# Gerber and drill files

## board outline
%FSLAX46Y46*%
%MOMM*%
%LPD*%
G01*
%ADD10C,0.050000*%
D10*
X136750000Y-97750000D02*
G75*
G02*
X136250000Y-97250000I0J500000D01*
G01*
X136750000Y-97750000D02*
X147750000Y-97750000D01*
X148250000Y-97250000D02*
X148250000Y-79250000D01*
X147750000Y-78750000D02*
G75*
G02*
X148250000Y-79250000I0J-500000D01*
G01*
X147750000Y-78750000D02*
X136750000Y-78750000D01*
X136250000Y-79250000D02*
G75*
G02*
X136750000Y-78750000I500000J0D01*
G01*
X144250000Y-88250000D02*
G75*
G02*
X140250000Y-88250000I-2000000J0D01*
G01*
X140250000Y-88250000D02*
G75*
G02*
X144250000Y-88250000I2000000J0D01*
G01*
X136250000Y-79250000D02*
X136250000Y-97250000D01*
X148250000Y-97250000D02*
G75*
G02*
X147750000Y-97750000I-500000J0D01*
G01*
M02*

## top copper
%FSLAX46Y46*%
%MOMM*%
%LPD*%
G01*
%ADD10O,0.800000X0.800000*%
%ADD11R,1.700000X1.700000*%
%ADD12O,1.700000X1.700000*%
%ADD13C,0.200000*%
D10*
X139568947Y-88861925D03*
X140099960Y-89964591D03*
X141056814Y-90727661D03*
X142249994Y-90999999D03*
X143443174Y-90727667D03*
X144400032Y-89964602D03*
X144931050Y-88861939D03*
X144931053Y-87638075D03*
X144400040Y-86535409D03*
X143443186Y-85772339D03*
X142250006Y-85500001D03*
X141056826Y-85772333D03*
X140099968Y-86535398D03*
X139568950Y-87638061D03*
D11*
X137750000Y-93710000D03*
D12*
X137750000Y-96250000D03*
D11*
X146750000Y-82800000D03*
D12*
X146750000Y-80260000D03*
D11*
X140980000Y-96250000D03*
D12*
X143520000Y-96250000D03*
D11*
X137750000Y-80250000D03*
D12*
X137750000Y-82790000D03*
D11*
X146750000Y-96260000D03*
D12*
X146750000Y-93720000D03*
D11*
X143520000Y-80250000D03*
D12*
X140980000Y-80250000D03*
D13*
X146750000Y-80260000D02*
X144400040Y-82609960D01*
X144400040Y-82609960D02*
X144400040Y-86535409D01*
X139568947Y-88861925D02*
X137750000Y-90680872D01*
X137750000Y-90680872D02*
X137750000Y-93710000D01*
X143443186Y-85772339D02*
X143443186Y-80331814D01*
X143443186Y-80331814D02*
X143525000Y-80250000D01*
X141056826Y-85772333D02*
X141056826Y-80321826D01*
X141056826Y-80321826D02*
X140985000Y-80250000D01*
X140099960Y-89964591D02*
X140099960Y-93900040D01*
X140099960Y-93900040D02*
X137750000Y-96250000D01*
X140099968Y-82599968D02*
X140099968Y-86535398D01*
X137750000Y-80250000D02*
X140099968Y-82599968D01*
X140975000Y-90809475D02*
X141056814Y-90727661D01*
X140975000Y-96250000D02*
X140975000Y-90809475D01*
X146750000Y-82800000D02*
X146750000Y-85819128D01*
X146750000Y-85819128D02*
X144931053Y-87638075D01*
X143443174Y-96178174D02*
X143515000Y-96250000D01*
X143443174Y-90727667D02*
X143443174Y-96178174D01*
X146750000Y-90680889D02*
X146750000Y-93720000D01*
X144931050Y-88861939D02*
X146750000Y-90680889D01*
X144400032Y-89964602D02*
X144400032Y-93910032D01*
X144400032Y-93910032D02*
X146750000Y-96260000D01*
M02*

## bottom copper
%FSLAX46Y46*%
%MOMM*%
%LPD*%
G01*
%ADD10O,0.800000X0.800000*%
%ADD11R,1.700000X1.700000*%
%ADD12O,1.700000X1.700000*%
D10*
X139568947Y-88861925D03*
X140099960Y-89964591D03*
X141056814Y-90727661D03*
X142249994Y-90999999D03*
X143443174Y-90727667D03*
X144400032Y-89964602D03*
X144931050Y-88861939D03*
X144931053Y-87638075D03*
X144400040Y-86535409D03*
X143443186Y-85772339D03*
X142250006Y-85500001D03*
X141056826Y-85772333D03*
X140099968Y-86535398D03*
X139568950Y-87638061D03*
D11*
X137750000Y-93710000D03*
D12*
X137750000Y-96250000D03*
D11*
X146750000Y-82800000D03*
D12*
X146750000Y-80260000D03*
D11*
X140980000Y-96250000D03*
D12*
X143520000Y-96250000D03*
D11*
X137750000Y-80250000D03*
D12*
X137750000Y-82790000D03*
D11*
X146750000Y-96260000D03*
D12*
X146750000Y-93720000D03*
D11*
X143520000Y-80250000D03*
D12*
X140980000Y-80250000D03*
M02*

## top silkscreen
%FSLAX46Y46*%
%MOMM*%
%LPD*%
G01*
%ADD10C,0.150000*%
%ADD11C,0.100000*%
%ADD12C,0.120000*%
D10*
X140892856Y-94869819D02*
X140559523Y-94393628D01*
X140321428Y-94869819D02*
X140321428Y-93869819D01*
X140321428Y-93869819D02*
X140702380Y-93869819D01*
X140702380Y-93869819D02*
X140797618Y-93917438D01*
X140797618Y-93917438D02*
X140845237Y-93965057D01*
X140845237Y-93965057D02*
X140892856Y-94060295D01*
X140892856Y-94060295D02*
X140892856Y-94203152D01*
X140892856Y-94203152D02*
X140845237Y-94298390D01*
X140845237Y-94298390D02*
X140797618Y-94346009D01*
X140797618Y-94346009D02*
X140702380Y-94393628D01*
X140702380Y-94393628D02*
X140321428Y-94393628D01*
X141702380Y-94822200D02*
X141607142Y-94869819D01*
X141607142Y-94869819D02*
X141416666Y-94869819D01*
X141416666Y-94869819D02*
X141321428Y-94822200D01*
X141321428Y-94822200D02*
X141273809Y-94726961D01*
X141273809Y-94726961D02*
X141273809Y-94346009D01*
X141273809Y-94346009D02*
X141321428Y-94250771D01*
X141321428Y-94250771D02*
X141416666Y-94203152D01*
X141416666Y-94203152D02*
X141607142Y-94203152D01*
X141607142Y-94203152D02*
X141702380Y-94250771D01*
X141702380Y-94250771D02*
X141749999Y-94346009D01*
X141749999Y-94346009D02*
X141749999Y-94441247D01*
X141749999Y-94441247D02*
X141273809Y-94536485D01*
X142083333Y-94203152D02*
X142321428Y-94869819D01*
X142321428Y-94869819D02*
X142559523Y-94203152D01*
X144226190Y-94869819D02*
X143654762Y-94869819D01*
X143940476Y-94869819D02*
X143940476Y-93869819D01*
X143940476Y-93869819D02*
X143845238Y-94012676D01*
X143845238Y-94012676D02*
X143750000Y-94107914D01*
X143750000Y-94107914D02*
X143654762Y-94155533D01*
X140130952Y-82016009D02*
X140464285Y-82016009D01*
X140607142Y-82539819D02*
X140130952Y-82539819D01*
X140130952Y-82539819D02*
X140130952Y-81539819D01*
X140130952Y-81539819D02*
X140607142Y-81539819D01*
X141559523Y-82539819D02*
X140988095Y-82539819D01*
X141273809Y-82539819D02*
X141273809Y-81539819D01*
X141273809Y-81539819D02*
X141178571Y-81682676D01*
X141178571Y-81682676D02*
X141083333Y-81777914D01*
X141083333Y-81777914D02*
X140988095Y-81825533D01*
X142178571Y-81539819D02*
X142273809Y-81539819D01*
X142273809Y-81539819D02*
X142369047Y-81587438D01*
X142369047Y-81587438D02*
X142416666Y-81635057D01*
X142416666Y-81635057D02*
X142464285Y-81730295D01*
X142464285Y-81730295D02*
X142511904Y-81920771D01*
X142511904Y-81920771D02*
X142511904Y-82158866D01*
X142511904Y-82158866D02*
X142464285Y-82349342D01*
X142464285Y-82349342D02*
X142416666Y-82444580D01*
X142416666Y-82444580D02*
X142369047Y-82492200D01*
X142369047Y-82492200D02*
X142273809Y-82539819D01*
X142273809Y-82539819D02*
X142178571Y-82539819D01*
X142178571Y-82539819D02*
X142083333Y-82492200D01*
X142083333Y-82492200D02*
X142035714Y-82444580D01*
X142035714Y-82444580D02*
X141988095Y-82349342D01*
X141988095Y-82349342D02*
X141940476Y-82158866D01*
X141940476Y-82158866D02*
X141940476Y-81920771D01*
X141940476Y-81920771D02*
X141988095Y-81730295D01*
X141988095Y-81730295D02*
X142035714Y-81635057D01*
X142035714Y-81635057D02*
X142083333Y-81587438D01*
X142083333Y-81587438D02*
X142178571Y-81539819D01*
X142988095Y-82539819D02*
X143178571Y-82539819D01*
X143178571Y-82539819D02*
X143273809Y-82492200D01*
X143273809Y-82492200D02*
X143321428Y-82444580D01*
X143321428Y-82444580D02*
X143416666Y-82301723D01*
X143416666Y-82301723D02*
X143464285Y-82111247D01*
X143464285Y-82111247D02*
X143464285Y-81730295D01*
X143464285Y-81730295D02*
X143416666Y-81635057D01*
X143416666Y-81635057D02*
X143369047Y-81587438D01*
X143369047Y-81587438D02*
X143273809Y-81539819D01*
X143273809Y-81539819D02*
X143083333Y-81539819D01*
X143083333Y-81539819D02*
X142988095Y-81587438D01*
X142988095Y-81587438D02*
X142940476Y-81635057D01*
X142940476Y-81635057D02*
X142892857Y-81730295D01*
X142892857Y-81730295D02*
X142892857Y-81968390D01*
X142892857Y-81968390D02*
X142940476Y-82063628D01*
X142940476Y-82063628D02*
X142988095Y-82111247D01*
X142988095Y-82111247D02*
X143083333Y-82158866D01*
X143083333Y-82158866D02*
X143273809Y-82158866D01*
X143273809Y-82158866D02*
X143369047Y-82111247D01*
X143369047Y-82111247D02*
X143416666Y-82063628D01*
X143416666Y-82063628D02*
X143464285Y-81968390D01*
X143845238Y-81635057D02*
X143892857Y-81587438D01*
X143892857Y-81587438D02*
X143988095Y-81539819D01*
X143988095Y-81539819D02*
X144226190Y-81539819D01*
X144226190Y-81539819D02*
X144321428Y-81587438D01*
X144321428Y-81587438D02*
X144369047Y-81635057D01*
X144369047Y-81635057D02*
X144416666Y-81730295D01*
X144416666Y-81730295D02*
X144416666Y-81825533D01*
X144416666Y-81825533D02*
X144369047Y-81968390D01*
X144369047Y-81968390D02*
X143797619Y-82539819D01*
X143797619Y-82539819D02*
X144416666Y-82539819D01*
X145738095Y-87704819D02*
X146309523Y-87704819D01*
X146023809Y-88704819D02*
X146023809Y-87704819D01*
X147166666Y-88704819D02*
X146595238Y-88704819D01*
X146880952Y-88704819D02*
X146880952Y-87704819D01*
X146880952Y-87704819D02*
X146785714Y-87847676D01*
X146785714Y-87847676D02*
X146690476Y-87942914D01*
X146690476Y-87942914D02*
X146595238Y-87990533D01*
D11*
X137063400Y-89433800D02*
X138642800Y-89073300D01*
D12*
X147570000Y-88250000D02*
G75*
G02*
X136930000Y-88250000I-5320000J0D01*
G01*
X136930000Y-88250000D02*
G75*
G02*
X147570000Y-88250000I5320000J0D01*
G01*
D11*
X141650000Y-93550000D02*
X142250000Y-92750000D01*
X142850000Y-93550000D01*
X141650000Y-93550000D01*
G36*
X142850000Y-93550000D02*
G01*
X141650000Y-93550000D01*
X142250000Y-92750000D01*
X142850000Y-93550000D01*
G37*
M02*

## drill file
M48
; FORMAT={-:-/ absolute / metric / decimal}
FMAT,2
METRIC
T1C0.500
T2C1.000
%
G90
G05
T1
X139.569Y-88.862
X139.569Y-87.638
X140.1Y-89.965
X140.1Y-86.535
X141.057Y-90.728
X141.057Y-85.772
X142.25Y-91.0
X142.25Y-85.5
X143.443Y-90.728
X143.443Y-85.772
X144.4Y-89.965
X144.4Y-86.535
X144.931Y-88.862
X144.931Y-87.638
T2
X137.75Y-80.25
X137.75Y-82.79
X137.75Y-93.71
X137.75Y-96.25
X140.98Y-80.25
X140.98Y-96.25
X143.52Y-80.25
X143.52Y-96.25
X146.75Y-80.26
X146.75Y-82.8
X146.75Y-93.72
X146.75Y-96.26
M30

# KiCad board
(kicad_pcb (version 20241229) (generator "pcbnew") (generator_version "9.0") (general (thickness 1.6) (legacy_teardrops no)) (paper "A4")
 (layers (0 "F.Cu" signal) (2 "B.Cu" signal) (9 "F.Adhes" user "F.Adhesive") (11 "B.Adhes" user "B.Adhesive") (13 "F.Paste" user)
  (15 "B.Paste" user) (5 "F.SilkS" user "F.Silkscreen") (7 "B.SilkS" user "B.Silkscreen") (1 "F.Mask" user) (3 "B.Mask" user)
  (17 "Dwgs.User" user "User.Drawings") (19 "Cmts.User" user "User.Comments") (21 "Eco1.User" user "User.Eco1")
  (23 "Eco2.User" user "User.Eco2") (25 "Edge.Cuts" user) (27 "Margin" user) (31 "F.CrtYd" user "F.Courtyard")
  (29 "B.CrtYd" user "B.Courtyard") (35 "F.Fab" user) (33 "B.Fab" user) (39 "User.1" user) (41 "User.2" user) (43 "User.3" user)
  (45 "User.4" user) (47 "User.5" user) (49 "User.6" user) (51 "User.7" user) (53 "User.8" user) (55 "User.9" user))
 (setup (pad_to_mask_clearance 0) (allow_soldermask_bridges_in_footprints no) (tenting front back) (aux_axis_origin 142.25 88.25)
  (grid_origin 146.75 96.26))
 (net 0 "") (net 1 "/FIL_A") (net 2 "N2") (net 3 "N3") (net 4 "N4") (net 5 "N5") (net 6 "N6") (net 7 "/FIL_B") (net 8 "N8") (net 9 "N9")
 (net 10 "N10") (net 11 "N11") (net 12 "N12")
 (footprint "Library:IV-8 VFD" (layer "F.Cu") (at 142.25 88.25)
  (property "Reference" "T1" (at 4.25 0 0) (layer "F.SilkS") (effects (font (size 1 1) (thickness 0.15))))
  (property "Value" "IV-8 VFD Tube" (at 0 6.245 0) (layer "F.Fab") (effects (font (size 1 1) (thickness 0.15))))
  (fp_line (start -5.1866 1.1838) (end -3.6072 0.8233) (stroke (width 0.1) (type default)) (layer "F.SilkS"))
  (fp_circle (center 0 0) (end 0 5.32) (stroke (width 0.12) (type default)) (fill no) (layer "F.SilkS"))
  (fp_poly (pts (xy -0.6 5.3) (xy 0 4.5) (xy 0.6 5.3)) (stroke (width 0.1) (type solid)) (fill yes) (layer "F.SilkS"))
  (pad "1" thru_hole oval (at -2.681053 0.611925) (size 0.8 0.8) (drill 0.5) (layers "*.Cu" "*.Mask") (remove_unused_layers no)
   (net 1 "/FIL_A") (thermal_bridge_angle 45))
  (pad "2" thru_hole oval (at -2.15004 1.714591) (size 0.8 0.8) (drill 0.5) (layers "*.Cu" "*.Mask") (remove_unused_layers no) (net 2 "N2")
   (thermal_bridge_angle 45))
  (pad "3" thru_hole oval (at -1.193186 2.477661) (size 0.8 0.8) (drill 0.5) (layers "*.Cu" "*.Mask") (remove_unused_layers no) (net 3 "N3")
   (thermal_bridge_angle 45))
  (pad "4" thru_hole oval (at -0.000006 2.749999) (size 0.8 0.8) (drill 0.5) (layers "*.Cu" "*.Mask") (remove_unused_layers no)
   (thermal_bridge_angle 45))
  (pad "5" thru_hole oval (at 1.193174 2.477667) (size 0.8 0.8) (drill 0.5) (layers "*.Cu" "*.Mask") (remove_unused_layers no) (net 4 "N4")
   (thermal_bridge_angle 45))
  (pad "6" thru_hole oval (at 2.150032 1.714602) (size 0.8 0.8) (drill 0.5) (layers "*.Cu" "*.Mask") (remove_unused_layers no) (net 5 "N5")
   (thermal_bridge_angle 45))
  (pad "7" thru_hole oval (at 2.68105 0.611939) (size 0.8 0.8) (drill 0.5) (layers "*.Cu" "*.Mask") (remove_unused_layers no) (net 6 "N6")
   (thermal_bridge_angle 45))
  (pad "8" thru_hole oval (at 2.681053 -0.611925) (size 0.8 0.8) (drill 0.5) (layers "*.Cu" "*.Mask") (remove_unused_layers no)
   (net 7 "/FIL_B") (thermal_bridge_angle 45))
  (pad "9" thru_hole oval (at 2.15004 -1.714591) (size 0.8 0.8) (drill 0.5) (layers "*.Cu" "*.Mask") (remove_unused_layers no) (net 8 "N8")
   (thermal_bridge_angle 45))
  (pad "10" thru_hole oval (at 1.193186 -2.477661) (size 0.8 0.8) (drill 0.5) (layers "*.Cu" "*.Mask") (remove_unused_layers no)
   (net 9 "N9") (thermal_bridge_angle 45))
  (pad "11" thru_hole oval (at 0.000006 -2.749999) (size 0.8 0.8) (drill 0.5) (layers "*.Cu" "*.Mask") (remove_unused_layers no)
   (thermal_bridge_angle 45))
  (pad "12" thru_hole oval (at -1.193174 -2.477667) (size 0.8 0.8) (drill 0.5) (layers "*.Cu" "*.Mask") (remove_unused_layers no)
   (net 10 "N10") (thermal_bridge_angle 45))
  (pad "13" thru_hole oval (at -2.150032 -1.714602) (size 0.8 0.8) (drill 0.5) (layers "*.Cu" "*.Mask") (remove_unused_layers no)
   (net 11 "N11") (thermal_bridge_angle 45))
  (pad "14" thru_hole oval (at -2.68105 -0.611939) (size 0.8 0.8) (drill 0.5) (layers "*.Cu" "*.Mask") (remove_unused_layers no)
   (thermal_bridge_angle 45)))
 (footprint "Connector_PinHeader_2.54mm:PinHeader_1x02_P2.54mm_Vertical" (layer "B.Cu") (at 137.75 93.71 180)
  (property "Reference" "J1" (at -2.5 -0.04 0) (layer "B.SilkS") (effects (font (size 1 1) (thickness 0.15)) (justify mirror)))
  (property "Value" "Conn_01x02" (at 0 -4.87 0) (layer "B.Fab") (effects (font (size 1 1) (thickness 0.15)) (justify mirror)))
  (pad "1" thru_hole rect (at 0 0 180) (size 1.7 1.7) (drill 1) (layers "*.Cu" "*.Mask") (remove_unused_layers no) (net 1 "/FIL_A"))
  (pad "2" thru_hole oval (at 0 -2.54 180) (size 1.7 1.7) (drill 1) (layers "*.Cu" "*.Mask") (remove_unused_layers no) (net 2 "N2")))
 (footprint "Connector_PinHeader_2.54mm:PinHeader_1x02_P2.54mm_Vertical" (layer "B.Cu") (at 146.75 82.8)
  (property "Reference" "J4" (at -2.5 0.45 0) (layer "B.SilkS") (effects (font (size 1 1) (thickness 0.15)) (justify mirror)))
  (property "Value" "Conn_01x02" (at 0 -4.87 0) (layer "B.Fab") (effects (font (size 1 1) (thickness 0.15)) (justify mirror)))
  (pad "1" thru_hole rect (at 0 0) (size 1.7 1.7) (drill 1) (layers "*.Cu" "*.Mask") (remove_unused_layers no) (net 7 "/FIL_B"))
  (pad "2" thru_hole oval (at 0 -2.54) (size 1.7 1.7) (drill 1) (layers "*.Cu" "*.Mask") (remove_unused_layers no) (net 8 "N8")))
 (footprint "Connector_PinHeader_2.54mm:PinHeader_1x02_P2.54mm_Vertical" (layer "B.Cu") (at 140.98 96.25 -90)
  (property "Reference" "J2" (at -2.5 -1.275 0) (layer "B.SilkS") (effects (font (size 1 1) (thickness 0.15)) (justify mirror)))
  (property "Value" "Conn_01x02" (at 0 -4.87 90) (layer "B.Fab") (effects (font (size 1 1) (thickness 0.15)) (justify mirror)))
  (pad "1" thru_hole rect (at 0 0 270) (size 1.7 1.7) (drill 1) (layers "*.Cu" "*.Mask") (remove_unused_layers no) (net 3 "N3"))
  (pad "2" thru_hole oval (at 0 -2.54 270) (size 1.7 1.7) (drill 1) (layers "*.Cu" "*.Mask") (remove_unused_layers no) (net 4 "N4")))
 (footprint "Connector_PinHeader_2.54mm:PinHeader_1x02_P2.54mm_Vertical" (layer "B.Cu") (at 137.75 80.25 180)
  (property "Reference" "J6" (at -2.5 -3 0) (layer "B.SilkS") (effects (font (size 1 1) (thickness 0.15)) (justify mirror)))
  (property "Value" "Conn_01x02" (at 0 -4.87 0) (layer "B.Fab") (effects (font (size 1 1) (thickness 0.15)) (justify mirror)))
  (pad "1" thru_hole rect (at 0 0 180) (size 1.7 1.7) (drill 1) (layers "*.Cu" "*.Mask") (remove_unused_layers no) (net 11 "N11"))
  (pad "2" thru_hole oval (at 0 -2.54 180) (size 1.7 1.7) (drill 1) (layers "*.Cu" "*.Mask") (remove_unused_layers no) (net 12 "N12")))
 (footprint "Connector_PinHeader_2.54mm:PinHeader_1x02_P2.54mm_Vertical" (layer "B.Cu") (at 146.75 96.26)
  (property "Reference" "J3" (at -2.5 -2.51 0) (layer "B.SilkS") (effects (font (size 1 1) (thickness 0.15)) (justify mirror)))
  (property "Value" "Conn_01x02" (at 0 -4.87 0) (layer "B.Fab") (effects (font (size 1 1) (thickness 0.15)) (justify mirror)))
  (pad "1" thru_hole rect (at 0 0) (size 1.7 1.7) (drill 1) (layers "*.Cu" "*.Mask") (remove_unused_layers no) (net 5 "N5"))
  (pad "2" thru_hole oval (at 0 -2.54) (size 1.7 1.7) (drill 1) (layers "*.Cu" "*.Mask") (remove_unused_layers no) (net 6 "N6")))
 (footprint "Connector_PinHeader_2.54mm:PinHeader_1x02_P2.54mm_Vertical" (layer "B.Cu") (at 143.52 80.25 90)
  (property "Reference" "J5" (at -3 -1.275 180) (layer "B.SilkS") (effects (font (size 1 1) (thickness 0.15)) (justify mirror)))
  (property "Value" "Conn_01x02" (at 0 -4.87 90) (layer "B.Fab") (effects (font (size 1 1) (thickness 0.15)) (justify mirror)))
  (pad "1" thru_hole rect (at 0 0 90) (size 1.7 1.7) (drill 1) (layers "*.Cu" "*.Mask") (remove_unused_layers no) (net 9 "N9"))
  (pad "2" thru_hole oval (at 0 -2.54 90) (size 1.7 1.7) (drill 1) (layers "*.Cu" "*.Mask") (remove_unused_layers no) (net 10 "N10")))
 (gr_arc (start 136.75 97.75) (mid 136.396447 97.603553) (end 136.25 97.25) (stroke (width 0.05) (type default)) (layer "Edge.Cuts"))
 (gr_line (start 136.75 97.75) (end 147.75 97.75) (stroke (width 0.05) (type default)) (layer "Edge.Cuts"))
 (gr_line (start 148.25 97.25) (end 148.25 79.25) (stroke (width 0.05) (type default)) (layer "Edge.Cuts"))
 (gr_arc (start 147.75 78.75) (mid 148.103553 78.896447) (end 148.25 79.25) (stroke (width 0.05) (type default)) (layer "Edge.Cuts"))
 (gr_line (start 147.75 78.75) (end 136.75 78.75) (stroke (width 0.05) (type default)) (layer "Edge.Cuts"))
 (gr_arc (start 136.25 79.25) (mid 136.396447 78.896447) (end 136.75 78.75) (stroke (width 0.05) (type default)) (layer "Edge.Cuts"))
 (gr_circle (center 142.25 88.25) (end 144.25 88.25) (stroke (width 0.05) (type solid)) (fill no) (layer "Edge.Cuts"))
 (gr_line (start 136.25 79.25) (end 136.25 97.25) (stroke (width 0.05) (type default)) (layer "Edge.Cuts"))
 (gr_arc (start 148.25 97.25) (mid 148.103553 97.603553) (end 147.75 97.75) (stroke (width 0.05) (type default)) (layer "Edge.Cuts"))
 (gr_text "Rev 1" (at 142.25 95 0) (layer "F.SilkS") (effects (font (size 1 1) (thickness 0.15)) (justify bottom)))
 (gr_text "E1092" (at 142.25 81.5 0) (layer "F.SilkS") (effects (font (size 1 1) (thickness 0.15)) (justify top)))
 (segment (start 146.75 80.26) (end 144.40004 82.60996) (width 0.2) (layer "F.Cu") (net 8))
 (segment (start 144.40004 82.60996) (end 144.40004 86.535409) (width 0.2) (layer "F.Cu") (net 8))
 (segment (start 139.568947 88.861925) (end 137.75 90.680872) (width 0.2) (layer "F.Cu") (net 1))
 (segment (start 137.75 90.680872) (end 137.75 93.71) (width 0.2) (layer "F.Cu") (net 1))
 (segment (start 143.443186 85.772339) (end 143.443186 80.331814) (width 0.2) (layer "F.Cu") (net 9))
 (segment (start 143.443186 80.331814) (end 143.525 80.25) (width 0.2) (layer "F.Cu") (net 9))
 (segment (start 141.056826 85.772333) (end 141.056826 80.321826) (width 0.2) (layer "F.Cu") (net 10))
 (segment (start 141.056826 80.321826) (end 140.985 80.25) (width 0.2) (layer "F.Cu") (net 10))
 (segment (start 140.09996 89.964591) (end 140.09996 93.90004) (width 0.2) (layer "F.Cu") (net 2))
 (segment (start 140.09996 93.90004) (end 137.75 96.25) (width 0.2) (layer "F.Cu") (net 2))
 (segment (start 140.099968 82.599968) (end 140.099968 86.535398) (width 0.2) (layer "F.Cu") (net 11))
 (segment (start 137.75 80.25) (end 140.099968 82.599968) (width 0.2) (layer "F.Cu") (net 11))
 (segment (start 140.975 90.809475) (end 141.056814 90.727661) (width 0.2) (layer "F.Cu") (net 3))
 (segment (start 140.975 96.25) (end 140.975 90.809475) (width 0.2) (layer "F.Cu") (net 3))
 (segment (start 146.75 82.8) (end 146.75 85.819128) (width 0.2) (layer "F.Cu") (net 7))
 (segment (start 146.75 85.819128) (end 144.931053 87.638075) (width 0.2) (layer "F.Cu") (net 7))
 (segment (start 143.443174 96.178174) (end 143.515 96.25) (width 0.2) (layer "F.Cu") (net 4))
 (segment (start 143.443174 90.727667) (end 143.443174 96.178174) (width 0.2) (layer "F.Cu") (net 4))
 (segment (start 146.75 90.680889) (end 146.75 93.72) (width 0.2) (layer "F.Cu") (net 6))
 (segment (start 144.93105 88.861939) (end 146.75 90.680889) (width 0.2) (layer "F.Cu") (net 6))
 (segment (start 144.400032 89.964602) (end 144.400032 93.910032) (width 0.2) (layer "F.Cu") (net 5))
 (segment (start 144.400032 93.910032) (end 146.75 96.26) (width 0.2) (layer "F.Cu") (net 5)))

